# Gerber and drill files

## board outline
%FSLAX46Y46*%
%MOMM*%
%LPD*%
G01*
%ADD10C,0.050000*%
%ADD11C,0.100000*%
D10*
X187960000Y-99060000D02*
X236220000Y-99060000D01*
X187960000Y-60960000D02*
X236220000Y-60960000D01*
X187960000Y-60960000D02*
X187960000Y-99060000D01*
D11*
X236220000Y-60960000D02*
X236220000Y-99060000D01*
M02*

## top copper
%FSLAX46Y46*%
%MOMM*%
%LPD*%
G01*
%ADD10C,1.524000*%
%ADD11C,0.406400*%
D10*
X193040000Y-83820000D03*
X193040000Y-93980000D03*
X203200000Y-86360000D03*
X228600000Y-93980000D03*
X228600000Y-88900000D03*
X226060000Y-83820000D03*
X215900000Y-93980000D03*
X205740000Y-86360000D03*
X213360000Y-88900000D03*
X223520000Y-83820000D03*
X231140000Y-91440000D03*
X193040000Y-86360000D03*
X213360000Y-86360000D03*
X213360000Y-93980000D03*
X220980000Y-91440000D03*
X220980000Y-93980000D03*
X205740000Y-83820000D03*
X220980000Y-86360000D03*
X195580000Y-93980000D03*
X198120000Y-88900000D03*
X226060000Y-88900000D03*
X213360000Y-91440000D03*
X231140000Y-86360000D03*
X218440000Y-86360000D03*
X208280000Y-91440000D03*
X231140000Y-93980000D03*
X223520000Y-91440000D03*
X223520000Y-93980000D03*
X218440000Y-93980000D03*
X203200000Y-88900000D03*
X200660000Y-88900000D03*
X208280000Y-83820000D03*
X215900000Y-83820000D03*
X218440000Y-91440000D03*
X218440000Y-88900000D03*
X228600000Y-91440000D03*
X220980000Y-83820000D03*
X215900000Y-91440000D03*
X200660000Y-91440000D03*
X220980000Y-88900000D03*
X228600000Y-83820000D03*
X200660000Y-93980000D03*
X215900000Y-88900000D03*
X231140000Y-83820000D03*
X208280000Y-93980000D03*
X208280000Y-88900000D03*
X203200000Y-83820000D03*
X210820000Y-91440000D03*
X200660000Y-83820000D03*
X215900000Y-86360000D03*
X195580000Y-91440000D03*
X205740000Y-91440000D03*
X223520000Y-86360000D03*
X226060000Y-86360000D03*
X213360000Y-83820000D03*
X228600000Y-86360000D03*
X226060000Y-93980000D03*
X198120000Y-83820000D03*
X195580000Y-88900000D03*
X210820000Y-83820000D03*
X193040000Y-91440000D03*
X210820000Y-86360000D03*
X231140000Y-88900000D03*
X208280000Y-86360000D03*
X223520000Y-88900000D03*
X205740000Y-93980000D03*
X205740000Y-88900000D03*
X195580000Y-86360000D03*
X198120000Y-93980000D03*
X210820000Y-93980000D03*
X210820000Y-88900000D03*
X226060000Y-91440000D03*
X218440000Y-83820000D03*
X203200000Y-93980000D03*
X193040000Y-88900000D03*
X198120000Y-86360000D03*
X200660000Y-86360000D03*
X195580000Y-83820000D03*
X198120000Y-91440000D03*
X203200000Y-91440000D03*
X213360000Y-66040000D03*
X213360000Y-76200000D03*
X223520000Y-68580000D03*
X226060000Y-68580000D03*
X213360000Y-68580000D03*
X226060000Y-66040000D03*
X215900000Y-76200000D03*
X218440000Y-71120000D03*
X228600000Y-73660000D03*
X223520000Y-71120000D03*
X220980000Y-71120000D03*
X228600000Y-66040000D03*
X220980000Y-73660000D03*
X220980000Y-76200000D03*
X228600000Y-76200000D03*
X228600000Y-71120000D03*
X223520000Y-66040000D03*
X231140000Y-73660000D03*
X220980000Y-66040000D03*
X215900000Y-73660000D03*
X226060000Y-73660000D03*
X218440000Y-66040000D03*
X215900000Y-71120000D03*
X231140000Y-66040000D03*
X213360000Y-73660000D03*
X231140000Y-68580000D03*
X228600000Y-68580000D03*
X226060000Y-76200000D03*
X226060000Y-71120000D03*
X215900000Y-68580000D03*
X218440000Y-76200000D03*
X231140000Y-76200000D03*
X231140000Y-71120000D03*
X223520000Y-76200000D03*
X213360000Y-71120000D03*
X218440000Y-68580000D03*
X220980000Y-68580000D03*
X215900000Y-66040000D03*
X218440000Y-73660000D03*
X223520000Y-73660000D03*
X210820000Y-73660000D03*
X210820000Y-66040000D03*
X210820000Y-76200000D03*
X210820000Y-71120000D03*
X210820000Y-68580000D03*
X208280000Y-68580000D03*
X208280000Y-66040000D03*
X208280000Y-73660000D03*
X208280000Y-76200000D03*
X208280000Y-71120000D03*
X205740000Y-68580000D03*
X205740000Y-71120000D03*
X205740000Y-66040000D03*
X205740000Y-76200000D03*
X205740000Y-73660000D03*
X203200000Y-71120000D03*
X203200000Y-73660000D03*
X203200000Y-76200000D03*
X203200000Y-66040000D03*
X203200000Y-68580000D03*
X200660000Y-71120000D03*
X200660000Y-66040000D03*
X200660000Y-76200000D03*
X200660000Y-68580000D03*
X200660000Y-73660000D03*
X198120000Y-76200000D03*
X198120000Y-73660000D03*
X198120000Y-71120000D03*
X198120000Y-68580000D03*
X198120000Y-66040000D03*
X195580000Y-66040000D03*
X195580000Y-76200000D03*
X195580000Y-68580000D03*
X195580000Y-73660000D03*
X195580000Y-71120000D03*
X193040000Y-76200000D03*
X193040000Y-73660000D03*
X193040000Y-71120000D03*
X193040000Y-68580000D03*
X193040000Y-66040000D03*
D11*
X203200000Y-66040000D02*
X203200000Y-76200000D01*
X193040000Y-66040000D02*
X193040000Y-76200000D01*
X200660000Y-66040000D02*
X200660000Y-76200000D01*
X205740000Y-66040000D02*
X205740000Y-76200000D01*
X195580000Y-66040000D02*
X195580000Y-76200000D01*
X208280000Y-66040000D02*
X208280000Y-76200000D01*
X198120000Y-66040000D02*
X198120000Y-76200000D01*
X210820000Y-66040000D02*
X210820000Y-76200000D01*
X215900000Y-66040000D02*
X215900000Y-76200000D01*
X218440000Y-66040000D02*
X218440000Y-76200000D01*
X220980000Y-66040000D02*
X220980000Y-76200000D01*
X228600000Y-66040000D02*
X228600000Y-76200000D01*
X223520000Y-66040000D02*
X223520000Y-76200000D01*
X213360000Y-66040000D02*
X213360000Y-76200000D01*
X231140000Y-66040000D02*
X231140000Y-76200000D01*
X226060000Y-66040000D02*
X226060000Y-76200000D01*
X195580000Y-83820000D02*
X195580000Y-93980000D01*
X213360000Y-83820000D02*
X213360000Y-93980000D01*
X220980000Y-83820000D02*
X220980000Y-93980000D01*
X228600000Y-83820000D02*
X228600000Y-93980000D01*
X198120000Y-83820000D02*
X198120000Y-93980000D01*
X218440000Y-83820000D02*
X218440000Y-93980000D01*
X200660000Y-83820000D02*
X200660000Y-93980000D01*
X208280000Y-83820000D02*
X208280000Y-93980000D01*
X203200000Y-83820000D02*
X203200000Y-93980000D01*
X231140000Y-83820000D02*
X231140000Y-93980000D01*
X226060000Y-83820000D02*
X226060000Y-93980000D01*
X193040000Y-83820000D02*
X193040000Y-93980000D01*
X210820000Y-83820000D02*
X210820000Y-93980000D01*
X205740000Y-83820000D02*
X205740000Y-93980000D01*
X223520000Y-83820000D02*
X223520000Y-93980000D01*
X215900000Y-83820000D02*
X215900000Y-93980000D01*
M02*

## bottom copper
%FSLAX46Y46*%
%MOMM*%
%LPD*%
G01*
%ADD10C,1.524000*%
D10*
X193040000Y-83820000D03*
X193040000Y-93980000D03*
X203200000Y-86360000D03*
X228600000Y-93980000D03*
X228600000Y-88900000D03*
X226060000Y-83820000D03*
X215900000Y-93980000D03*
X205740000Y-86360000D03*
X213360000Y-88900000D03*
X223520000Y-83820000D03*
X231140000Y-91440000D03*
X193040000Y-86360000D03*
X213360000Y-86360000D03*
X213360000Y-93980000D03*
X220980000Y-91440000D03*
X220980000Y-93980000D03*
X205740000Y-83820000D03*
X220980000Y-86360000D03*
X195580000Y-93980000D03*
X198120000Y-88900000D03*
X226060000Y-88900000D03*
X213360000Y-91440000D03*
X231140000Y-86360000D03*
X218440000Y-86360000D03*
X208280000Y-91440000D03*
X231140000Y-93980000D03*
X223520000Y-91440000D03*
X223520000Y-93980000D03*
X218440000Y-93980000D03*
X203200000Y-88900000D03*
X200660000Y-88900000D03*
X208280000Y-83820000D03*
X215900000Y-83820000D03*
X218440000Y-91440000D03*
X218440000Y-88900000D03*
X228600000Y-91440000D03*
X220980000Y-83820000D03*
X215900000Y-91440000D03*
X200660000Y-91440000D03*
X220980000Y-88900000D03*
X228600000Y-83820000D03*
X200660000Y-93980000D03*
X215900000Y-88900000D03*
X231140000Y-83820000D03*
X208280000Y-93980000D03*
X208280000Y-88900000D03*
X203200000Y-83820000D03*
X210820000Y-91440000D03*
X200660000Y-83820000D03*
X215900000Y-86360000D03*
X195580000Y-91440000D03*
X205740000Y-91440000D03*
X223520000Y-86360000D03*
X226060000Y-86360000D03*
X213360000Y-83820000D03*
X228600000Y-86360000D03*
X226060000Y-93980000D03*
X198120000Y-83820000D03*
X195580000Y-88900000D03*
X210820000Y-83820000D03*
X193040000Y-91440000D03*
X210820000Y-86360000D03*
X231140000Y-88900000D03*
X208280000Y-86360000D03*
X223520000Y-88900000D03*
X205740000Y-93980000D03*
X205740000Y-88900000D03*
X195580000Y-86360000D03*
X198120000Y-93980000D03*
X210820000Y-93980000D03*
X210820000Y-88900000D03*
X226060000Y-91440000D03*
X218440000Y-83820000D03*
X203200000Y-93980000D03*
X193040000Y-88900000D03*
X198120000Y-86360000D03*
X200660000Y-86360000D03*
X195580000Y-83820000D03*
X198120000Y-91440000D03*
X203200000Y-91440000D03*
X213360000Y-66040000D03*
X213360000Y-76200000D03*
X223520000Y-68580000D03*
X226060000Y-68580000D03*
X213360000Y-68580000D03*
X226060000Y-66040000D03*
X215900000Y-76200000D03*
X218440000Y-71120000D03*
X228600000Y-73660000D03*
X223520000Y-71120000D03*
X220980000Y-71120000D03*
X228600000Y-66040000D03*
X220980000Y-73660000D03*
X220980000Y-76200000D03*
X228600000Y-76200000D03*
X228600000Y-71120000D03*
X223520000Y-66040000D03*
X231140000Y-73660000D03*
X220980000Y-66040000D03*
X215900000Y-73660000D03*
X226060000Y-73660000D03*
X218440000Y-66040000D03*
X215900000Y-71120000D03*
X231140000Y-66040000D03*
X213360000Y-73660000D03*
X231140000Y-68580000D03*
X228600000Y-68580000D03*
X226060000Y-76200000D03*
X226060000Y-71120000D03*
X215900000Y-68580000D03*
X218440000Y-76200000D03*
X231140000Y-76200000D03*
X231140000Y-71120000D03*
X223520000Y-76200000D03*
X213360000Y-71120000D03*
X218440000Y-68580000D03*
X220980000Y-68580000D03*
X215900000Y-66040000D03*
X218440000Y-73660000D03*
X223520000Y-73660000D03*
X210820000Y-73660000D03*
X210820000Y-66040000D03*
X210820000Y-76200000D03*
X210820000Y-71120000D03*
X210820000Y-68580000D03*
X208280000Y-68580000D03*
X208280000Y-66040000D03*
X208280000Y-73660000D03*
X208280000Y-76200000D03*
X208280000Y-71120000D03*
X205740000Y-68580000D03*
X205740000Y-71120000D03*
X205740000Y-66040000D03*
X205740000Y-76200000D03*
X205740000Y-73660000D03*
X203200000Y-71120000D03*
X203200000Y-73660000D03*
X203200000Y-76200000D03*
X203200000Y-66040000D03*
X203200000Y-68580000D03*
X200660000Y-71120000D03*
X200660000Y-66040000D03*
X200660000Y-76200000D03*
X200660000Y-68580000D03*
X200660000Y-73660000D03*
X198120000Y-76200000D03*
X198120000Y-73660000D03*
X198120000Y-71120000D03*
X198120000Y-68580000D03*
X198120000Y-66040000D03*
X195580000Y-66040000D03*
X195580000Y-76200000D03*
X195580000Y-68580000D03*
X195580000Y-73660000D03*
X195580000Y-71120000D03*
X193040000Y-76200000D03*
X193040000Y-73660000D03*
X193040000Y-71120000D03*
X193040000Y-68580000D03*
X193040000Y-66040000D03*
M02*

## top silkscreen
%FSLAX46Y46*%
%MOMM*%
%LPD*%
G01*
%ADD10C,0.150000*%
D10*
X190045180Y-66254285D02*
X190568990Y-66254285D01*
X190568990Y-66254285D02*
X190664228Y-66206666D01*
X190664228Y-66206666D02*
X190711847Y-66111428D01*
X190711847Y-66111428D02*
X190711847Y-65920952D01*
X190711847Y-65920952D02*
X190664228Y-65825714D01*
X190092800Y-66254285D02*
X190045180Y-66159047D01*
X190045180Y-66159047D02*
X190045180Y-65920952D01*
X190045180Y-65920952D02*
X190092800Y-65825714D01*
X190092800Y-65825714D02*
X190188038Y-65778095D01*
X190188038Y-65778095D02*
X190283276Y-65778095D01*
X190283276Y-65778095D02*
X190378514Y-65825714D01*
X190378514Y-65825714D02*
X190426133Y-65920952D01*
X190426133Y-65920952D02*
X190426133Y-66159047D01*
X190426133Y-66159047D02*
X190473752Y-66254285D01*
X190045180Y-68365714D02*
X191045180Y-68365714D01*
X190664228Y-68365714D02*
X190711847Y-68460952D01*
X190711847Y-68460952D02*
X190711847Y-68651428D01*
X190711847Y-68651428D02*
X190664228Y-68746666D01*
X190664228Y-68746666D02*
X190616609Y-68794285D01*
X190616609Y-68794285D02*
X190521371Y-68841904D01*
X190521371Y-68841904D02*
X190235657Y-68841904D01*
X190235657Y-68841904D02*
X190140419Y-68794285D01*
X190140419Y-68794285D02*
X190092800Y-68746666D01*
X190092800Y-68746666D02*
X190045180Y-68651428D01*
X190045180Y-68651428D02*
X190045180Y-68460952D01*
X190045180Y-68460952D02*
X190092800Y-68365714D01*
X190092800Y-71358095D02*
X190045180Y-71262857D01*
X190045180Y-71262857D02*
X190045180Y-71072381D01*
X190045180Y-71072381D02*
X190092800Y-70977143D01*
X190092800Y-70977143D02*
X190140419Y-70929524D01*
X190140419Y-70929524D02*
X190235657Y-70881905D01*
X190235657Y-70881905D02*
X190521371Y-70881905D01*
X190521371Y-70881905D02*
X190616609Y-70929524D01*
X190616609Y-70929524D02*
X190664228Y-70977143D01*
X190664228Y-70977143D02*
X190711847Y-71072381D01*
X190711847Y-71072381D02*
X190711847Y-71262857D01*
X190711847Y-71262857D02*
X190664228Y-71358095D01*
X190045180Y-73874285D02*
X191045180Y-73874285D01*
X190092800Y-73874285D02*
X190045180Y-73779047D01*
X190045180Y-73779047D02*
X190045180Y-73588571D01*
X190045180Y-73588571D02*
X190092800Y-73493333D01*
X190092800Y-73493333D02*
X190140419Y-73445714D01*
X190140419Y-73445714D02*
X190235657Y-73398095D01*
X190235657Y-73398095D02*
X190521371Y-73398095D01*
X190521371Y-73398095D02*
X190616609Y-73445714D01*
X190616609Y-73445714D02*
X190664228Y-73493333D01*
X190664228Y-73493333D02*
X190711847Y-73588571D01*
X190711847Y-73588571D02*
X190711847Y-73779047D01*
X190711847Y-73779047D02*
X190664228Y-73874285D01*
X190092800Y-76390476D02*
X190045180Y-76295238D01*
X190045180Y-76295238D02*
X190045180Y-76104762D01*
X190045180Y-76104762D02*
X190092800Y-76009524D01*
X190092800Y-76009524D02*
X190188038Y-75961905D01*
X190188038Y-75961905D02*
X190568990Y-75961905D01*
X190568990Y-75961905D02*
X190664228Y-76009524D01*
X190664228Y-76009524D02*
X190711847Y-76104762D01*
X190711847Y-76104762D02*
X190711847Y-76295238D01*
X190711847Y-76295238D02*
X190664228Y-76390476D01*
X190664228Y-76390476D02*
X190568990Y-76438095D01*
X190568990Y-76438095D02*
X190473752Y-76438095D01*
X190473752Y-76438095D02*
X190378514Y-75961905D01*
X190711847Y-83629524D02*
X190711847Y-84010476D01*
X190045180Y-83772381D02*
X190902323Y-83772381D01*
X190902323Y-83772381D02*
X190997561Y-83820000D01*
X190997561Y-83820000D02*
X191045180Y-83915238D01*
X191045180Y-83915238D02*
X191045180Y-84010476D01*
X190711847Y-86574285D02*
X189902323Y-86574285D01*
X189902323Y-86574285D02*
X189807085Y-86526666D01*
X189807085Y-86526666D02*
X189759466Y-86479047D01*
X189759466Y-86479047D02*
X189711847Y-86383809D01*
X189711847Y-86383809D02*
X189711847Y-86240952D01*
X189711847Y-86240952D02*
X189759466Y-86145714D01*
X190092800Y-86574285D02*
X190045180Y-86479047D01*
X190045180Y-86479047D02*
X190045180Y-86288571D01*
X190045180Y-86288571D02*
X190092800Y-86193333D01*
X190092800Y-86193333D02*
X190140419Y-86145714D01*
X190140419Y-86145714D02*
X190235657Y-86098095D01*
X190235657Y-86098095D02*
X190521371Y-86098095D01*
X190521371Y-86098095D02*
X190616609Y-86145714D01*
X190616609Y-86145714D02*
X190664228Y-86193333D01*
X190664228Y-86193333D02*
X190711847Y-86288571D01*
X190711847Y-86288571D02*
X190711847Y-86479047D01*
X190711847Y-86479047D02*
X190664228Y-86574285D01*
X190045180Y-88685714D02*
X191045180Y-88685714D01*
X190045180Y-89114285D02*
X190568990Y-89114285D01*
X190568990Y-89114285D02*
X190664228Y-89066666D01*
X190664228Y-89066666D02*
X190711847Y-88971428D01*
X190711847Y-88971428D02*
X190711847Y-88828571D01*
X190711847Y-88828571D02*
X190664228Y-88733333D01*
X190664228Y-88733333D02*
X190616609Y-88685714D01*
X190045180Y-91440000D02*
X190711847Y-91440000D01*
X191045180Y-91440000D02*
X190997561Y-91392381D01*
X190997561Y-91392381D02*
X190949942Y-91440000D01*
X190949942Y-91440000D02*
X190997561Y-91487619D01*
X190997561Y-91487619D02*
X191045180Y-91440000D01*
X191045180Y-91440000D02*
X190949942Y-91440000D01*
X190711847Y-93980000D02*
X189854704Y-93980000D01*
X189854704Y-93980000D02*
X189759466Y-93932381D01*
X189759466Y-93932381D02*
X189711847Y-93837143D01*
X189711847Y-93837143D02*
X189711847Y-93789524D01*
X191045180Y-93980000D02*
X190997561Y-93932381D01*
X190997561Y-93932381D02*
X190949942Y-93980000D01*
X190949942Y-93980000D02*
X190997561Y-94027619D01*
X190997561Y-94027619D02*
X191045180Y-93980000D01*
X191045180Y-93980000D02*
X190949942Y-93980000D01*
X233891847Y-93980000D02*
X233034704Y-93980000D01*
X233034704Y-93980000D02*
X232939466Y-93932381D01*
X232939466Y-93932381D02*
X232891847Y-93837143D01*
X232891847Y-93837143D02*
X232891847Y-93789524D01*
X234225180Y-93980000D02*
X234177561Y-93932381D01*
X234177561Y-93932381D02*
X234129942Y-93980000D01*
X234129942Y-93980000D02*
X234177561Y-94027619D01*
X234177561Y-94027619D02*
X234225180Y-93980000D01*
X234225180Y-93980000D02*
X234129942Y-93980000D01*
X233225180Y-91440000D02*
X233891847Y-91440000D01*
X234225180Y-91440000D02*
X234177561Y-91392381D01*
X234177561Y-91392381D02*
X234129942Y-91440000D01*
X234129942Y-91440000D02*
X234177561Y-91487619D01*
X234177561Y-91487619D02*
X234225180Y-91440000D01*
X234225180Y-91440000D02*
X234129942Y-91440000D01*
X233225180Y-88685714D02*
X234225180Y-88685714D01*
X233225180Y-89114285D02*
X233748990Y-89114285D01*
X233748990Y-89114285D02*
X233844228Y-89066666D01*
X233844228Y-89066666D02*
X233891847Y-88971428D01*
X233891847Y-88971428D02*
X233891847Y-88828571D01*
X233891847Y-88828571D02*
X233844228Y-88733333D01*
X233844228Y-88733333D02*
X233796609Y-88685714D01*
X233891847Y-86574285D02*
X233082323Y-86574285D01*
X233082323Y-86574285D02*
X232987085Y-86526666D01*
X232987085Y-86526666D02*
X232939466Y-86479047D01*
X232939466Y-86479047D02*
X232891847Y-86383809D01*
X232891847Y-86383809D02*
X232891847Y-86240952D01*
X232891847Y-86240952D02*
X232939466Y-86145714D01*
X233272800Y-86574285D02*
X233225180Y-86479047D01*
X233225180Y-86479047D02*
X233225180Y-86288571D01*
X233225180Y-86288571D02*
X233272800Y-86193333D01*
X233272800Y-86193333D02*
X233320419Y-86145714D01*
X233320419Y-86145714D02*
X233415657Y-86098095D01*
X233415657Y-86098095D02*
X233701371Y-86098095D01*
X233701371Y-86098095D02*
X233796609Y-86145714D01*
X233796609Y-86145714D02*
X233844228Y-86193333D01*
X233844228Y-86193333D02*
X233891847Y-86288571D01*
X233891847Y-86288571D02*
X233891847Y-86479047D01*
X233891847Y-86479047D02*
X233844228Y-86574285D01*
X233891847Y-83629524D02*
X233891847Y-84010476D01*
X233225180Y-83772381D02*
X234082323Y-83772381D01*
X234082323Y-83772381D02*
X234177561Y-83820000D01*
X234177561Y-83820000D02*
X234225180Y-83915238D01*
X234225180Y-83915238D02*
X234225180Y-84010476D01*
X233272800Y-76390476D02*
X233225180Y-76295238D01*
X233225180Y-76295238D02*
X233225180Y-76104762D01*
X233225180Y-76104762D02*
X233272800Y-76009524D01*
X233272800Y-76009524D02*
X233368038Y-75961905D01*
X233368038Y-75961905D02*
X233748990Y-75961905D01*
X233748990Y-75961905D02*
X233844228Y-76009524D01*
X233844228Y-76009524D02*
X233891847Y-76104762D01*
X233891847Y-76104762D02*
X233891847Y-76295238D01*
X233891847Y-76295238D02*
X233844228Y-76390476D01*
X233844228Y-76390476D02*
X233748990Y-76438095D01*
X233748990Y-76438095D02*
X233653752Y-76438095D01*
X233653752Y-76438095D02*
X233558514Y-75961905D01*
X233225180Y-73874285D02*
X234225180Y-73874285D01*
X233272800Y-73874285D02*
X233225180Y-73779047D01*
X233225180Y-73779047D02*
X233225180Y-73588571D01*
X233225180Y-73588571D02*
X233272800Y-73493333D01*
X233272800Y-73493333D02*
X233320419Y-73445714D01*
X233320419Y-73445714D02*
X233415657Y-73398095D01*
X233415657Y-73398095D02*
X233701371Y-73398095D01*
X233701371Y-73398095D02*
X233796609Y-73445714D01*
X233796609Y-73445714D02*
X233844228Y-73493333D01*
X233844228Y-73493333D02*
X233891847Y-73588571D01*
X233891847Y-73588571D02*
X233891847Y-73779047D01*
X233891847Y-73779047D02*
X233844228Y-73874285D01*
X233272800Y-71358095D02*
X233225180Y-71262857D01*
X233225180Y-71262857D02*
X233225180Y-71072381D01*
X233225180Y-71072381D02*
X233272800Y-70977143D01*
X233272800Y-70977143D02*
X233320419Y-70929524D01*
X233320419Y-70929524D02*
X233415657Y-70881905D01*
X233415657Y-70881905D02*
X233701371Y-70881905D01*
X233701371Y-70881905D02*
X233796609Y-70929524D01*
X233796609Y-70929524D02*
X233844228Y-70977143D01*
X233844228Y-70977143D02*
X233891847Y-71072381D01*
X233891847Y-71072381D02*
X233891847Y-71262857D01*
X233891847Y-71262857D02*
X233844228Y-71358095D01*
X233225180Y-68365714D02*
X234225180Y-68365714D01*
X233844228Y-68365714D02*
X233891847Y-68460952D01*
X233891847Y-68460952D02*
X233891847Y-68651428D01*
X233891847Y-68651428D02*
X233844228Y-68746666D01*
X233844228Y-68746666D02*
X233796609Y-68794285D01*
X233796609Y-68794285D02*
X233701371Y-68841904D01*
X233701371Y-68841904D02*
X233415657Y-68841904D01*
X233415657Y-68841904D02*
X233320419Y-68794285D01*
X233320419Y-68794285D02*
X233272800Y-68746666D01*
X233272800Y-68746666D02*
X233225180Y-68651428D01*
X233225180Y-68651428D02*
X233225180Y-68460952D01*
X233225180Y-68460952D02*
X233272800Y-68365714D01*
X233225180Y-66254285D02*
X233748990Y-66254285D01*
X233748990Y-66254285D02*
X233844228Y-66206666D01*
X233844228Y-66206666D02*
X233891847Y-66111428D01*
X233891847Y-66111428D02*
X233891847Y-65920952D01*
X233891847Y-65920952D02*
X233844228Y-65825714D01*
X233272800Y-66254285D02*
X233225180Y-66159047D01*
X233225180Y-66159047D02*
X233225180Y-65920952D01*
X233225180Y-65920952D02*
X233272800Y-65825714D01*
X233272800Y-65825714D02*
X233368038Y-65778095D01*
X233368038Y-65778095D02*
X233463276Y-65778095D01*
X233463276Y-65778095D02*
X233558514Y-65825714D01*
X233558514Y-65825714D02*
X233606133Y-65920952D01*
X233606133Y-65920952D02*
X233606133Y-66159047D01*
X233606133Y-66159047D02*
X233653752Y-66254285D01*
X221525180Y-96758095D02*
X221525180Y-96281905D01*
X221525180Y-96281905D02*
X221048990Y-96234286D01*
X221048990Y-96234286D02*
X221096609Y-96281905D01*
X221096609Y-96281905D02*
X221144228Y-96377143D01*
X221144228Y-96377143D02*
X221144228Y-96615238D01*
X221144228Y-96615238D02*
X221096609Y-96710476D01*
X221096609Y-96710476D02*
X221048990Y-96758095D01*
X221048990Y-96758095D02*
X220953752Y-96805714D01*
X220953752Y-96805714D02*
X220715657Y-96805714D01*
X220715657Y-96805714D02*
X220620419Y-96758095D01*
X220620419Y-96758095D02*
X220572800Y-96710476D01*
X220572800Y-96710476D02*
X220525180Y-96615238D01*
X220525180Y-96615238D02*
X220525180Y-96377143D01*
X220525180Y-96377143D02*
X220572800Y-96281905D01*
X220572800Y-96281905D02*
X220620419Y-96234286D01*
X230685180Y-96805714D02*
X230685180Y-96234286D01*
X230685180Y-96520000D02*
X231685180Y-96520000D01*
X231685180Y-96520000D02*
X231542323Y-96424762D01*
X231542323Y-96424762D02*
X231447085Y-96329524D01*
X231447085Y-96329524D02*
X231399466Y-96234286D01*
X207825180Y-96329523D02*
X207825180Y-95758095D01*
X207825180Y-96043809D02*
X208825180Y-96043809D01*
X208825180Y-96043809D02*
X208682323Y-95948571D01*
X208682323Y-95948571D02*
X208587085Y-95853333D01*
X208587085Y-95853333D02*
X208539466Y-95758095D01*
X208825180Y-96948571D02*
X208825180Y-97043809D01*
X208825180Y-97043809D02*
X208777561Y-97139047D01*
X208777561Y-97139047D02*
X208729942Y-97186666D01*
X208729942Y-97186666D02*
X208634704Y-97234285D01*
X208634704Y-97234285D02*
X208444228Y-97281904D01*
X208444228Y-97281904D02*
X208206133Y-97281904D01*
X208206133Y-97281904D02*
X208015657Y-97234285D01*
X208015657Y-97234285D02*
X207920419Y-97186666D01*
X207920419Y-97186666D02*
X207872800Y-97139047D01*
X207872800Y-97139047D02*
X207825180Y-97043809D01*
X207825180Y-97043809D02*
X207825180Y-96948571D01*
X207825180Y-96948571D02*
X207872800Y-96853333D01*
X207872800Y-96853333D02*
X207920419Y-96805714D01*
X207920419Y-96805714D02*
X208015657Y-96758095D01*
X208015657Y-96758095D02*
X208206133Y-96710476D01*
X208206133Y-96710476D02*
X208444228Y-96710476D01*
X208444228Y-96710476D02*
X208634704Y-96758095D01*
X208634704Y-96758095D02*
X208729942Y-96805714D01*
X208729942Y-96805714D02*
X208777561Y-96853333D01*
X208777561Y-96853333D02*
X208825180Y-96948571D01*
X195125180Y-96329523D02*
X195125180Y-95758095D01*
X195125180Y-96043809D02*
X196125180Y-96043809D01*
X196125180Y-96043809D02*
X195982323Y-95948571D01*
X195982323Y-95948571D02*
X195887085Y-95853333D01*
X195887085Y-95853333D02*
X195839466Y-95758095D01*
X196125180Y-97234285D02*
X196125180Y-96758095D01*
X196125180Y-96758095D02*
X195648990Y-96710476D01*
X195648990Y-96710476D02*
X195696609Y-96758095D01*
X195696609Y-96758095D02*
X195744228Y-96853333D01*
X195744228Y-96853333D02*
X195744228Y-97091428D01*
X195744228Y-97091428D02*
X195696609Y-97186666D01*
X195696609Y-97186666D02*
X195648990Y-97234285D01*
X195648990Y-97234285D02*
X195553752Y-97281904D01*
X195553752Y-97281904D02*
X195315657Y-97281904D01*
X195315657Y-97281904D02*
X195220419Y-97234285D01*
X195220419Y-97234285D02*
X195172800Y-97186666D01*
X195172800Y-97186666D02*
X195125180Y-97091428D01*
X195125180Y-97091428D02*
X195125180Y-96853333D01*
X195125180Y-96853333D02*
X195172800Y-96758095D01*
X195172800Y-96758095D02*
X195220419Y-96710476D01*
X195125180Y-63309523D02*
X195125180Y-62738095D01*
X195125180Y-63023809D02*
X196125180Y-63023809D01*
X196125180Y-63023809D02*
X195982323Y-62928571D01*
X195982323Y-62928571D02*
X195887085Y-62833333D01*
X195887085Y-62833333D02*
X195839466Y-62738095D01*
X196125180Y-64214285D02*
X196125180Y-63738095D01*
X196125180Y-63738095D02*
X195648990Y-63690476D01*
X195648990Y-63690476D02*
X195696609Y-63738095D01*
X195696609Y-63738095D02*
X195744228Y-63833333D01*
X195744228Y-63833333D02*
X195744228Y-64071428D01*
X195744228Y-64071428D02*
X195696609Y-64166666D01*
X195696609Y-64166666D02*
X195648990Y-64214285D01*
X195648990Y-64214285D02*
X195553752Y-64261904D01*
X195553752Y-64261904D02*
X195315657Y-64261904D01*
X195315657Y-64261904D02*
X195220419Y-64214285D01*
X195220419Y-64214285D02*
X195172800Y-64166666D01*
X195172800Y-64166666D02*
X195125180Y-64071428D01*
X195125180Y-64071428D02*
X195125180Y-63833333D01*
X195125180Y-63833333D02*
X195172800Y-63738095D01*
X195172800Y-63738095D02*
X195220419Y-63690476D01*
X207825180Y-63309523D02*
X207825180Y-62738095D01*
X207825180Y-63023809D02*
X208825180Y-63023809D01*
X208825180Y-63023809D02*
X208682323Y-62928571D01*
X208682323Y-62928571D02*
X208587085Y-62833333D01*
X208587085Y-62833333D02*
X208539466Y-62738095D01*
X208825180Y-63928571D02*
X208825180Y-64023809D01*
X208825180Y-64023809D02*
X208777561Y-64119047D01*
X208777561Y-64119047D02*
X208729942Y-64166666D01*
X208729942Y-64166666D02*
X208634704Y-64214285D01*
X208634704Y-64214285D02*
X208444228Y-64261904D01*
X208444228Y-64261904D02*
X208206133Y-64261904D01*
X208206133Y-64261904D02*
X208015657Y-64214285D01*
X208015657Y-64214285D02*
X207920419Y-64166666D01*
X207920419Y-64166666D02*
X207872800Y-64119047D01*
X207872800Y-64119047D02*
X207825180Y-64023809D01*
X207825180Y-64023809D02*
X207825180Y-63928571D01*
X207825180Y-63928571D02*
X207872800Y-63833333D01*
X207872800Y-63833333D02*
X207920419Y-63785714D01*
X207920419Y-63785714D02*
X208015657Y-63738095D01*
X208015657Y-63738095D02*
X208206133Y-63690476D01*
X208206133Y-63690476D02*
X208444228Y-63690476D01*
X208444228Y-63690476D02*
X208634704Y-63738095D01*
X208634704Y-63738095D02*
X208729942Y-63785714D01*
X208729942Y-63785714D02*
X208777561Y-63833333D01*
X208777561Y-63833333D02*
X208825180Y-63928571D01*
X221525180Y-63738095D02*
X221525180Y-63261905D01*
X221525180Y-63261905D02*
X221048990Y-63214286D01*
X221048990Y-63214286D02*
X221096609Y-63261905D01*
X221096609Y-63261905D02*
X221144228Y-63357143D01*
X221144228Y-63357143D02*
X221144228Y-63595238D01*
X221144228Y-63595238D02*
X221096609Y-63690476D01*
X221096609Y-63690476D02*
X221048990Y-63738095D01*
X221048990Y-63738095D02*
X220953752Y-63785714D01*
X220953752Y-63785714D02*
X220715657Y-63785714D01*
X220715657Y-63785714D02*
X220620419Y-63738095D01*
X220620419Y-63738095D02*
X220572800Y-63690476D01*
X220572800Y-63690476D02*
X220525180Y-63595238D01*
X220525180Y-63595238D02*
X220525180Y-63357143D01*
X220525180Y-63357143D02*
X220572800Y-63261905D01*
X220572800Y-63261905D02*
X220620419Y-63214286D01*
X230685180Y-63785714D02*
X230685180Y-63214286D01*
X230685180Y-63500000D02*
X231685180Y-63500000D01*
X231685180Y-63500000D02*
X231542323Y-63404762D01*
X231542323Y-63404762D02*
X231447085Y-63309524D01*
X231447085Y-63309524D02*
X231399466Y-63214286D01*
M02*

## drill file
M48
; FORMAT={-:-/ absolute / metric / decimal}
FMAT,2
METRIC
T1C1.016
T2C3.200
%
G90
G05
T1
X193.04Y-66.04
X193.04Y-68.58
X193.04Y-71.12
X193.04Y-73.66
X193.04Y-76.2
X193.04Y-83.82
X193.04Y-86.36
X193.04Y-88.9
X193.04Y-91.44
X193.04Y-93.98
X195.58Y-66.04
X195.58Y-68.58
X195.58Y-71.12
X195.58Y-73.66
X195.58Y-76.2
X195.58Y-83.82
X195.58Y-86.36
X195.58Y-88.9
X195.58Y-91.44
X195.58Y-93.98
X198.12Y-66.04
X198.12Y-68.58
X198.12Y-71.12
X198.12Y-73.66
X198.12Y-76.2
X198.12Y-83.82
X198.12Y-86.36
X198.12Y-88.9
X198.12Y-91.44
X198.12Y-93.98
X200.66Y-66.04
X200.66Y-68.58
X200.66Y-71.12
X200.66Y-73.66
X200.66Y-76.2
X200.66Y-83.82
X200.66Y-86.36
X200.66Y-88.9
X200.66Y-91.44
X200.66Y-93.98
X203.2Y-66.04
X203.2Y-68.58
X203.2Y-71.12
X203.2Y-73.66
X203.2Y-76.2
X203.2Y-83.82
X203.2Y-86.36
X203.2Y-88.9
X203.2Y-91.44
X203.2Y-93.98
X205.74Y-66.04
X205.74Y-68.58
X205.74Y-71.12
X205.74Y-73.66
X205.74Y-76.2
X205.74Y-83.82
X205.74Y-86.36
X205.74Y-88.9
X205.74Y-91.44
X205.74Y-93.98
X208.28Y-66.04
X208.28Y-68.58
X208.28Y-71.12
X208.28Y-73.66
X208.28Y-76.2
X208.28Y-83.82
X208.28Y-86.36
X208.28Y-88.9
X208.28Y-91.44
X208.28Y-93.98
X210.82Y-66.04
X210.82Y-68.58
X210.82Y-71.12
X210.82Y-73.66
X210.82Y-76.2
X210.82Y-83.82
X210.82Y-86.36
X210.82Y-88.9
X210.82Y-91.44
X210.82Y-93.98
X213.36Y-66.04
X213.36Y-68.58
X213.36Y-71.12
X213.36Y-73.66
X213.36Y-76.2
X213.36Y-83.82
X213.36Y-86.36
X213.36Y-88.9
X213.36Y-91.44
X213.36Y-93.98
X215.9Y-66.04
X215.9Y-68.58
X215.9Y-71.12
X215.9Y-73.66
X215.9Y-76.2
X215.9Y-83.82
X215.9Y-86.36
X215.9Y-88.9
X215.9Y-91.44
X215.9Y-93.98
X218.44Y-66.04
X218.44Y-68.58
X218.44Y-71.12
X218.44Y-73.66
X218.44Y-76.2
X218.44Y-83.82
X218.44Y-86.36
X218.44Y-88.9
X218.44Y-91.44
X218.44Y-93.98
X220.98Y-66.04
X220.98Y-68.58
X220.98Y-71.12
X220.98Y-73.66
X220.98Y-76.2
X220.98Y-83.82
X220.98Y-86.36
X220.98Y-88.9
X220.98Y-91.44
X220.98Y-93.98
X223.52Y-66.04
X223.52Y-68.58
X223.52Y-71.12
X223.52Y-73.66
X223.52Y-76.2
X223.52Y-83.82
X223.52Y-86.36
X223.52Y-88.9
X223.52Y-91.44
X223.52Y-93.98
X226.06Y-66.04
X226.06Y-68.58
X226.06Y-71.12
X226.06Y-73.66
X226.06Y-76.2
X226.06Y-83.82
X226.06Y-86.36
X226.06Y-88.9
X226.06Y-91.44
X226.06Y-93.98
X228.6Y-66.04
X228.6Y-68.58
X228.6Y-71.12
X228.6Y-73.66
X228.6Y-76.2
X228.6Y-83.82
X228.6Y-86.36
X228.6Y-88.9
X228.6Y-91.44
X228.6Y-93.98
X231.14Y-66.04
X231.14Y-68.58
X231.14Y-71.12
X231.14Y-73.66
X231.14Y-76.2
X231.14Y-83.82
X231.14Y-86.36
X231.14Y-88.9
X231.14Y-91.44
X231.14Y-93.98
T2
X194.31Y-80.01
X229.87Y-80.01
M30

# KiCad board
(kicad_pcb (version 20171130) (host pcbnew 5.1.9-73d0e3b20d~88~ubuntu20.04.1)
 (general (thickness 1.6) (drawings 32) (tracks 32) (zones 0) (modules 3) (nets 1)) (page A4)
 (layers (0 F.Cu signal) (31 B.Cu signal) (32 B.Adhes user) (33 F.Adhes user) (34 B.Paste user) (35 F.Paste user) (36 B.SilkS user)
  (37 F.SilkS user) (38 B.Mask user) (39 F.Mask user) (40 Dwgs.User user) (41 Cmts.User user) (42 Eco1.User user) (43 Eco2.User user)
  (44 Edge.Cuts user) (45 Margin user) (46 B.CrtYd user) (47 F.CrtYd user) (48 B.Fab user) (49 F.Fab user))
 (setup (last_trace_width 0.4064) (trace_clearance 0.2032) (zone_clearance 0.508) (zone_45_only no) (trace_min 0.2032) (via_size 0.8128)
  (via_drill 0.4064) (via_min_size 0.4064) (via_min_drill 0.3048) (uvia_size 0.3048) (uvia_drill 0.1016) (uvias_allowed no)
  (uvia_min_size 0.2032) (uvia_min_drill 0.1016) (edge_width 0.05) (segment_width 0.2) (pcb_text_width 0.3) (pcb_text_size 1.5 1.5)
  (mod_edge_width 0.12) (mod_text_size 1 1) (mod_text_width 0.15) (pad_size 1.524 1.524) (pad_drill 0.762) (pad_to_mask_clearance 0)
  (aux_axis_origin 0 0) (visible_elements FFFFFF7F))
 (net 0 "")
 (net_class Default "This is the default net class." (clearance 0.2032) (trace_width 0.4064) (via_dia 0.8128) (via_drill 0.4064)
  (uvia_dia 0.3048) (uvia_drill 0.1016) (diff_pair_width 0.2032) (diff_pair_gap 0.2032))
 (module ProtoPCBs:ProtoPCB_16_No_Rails (layer F.Cu) (at 193.04 66.04)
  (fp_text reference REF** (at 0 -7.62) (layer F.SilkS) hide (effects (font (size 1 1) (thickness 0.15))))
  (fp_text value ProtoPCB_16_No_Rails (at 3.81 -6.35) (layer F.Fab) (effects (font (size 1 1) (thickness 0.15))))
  (pad 1 thru_hole circle (at 0 17.78) (size 1.524 1.524) (drill 1.016) (layers *.Cu *.Mask))
  (pad 1 thru_hole circle (at 0 27.94) (size 1.524 1.524) (drill 1.016) (layers *.Cu *.Mask))
  (pad 1 thru_hole circle (at 10.16 20.32) (size 1.524 1.524) (drill 1.016) (layers *.Cu *.Mask))
  (pad 1 thru_hole circle (at 35.56 27.94) (size 1.524 1.524) (drill 1.016) (layers *.Cu *.Mask))
  (pad 1 thru_hole circle (at 35.56 22.86) (size 1.524 1.524) (drill 1.016) (layers *.Cu *.Mask))
  (pad 1 thru_hole circle (at 33.02 17.78) (size 1.524 1.524) (drill 1.016) (layers *.Cu *.Mask))
  (pad 1 thru_hole circle (at 22.86 27.94) (size 1.524 1.524) (drill 1.016) (layers *.Cu *.Mask))
  (pad 1 thru_hole circle (at 12.7 20.32) (size 1.524 1.524) (drill 1.016) (layers *.Cu *.Mask))
  (pad 1 thru_hole circle (at 20.32 22.86) (size 1.524 1.524) (drill 1.016) (layers *.Cu *.Mask))
  (pad 1 thru_hole circle (at 30.48 17.78) (size 1.524 1.524) (drill 1.016) (layers *.Cu *.Mask))
  (pad 1 thru_hole circle (at 38.1 25.4) (size 1.524 1.524) (drill 1.016) (layers *.Cu *.Mask))
  (pad 1 thru_hole circle (at 0 20.32) (size 1.524 1.524) (drill 1.016) (layers *.Cu *.Mask))
  (pad 1 thru_hole circle (at 20.32 20.32) (size 1.524 1.524) (drill 1.016) (layers *.Cu *.Mask))
  (pad 1 thru_hole circle (at 20.32 27.94) (size 1.524 1.524) (drill 1.016) (layers *.Cu *.Mask))
  (pad 1 thru_hole circle (at 27.94 25.4) (size 1.524 1.524) (drill 1.016) (layers *.Cu *.Mask))
  (pad 1 thru_hole circle (at 27.94 27.94) (size 1.524 1.524) (drill 1.016) (layers *.Cu *.Mask))
  (pad 1 thru_hole circle (at 12.7 17.78) (size 1.524 1.524) (drill 1.016) (layers *.Cu *.Mask))
  (pad 1 thru_hole circle (at 27.94 20.32) (size 1.524 1.524) (drill 1.016) (layers *.Cu *.Mask))
  (pad 1 thru_hole circle (at 2.54 27.94) (size 1.524 1.524) (drill 1.016) (layers *.Cu *.Mask))
  (pad 1 thru_hole circle (at 5.08 22.86) (size 1.524 1.524) (drill 1.016) (layers *.Cu *.Mask))
  (pad 1 thru_hole circle (at 33.02 22.86) (size 1.524 1.524) (drill 1.016) (layers *.Cu *.Mask))
  (pad 1 thru_hole circle (at 20.32 25.4) (size 1.524 1.524) (drill 1.016) (layers *.Cu *.Mask))
  (pad 1 thru_hole circle (at 38.1 20.32) (size 1.524 1.524) (drill 1.016) (layers *.Cu *.Mask))
  (pad 1 thru_hole circle (at 25.4 20.32) (size 1.524 1.524) (drill 1.016) (layers *.Cu *.Mask))
  (pad 1 thru_hole circle (at 15.24 25.4) (size 1.524 1.524) (drill 1.016) (layers *.Cu *.Mask))
  (pad 1 thru_hole circle (at 38.1 27.94) (size 1.524 1.524) (drill 1.016) (layers *.Cu *.Mask))
  (pad 1 thru_hole circle (at 30.48 25.4) (size 1.524 1.524) (drill 1.016) (layers *.Cu *.Mask))
  (pad 1 thru_hole circle (at 30.48 27.94) (size 1.524 1.524) (drill 1.016) (layers *.Cu *.Mask))
  (pad 1 thru_hole circle (at 25.4 27.94) (size 1.524 1.524) (drill 1.016) (layers *.Cu *.Mask))
  (pad 1 thru_hole circle (at 10.16 22.86) (size 1.524 1.524) (drill 1.016) (layers *.Cu *.Mask))
  (pad 1 thru_hole circle (at 7.62 22.86) (size 1.524 1.524) (drill 1.016) (layers *.Cu *.Mask))
  (pad 1 thru_hole circle (at 15.24 17.78) (size 1.524 1.524) (drill 1.016) (layers *.Cu *.Mask))
  (pad 1 thru_hole circle (at 22.86 17.78) (size 1.524 1.524) (drill 1.016) (layers *.Cu *.Mask))
  (pad 1 thru_hole circle (at 25.4 25.4) (size 1.524 1.524) (drill 1.016) (layers *.Cu *.Mask))
  (pad 1 thru_hole circle (at 25.4 22.86) (size 1.524 1.524) (drill 1.016) (layers *.Cu *.Mask))
  (pad 1 thru_hole circle (at 35.56 25.4) (size 1.524 1.524) (drill 1.016) (layers *.Cu *.Mask))
  (pad 1 thru_hole circle (at 27.94 17.78) (size 1.524 1.524) (drill 1.016) (layers *.Cu *.Mask))
  (pad 1 thru_hole circle (at 22.86 25.4) (size 1.524 1.524) (drill 1.016) (layers *.Cu *.Mask))
  (pad 1 thru_hole circle (at 7.62 25.4) (size 1.524 1.524) (drill 1.016) (layers *.Cu *.Mask))
  (pad 1 thru_hole circle (at 27.94 22.86) (size 1.524 1.524) (drill 1.016) (layers *.Cu *.Mask))
  (pad 1 thru_hole circle (at 35.56 17.78) (size 1.524 1.524) (drill 1.016) (layers *.Cu *.Mask))
  (pad 1 thru_hole circle (at 7.62 27.94) (size 1.524 1.524) (drill 1.016) (layers *.Cu *.Mask))
  (pad 1 thru_hole circle (at 22.86 22.86) (size 1.524 1.524) (drill 1.016) (layers *.Cu *.Mask))
  (pad 1 thru_hole circle (at 38.1 17.78) (size 1.524 1.524) (drill 1.016) (layers *.Cu *.Mask))
  (pad 1 thru_hole circle (at 15.24 27.94) (size 1.524 1.524) (drill 1.016) (layers *.Cu *.Mask))
  (pad 1 thru_hole circle (at 15.24 22.86) (size 1.524 1.524) (drill 1.016) (layers *.Cu *.Mask))
  (pad 1 thru_hole circle (at 10.16 17.78) (size 1.524 1.524) (drill 1.016) (layers *.Cu *.Mask))
  (pad 1 thru_hole circle (at 17.78 25.4) (size 1.524 1.524) (drill 1.016) (layers *.Cu *.Mask))
  (pad 1 thru_hole circle (at 7.62 17.78) (size 1.524 1.524) (drill 1.016) (layers *.Cu *.Mask))
  (pad 1 thru_hole circle (at 22.86 20.32) (size 1.524 1.524) (drill 1.016) (layers *.Cu *.Mask))
  (pad 1 thru_hole circle (at 2.54 25.4) (size 1.524 1.524) (drill 1.016) (layers *.Cu *.Mask))
  (pad 1 thru_hole circle (at 12.7 25.4) (size 1.524 1.524) (drill 1.016) (layers *.Cu *.Mask))
  (pad 1 thru_hole circle (at 30.48 20.32) (size 1.524 1.524) (drill 1.016) (layers *.Cu *.Mask))
  (pad 1 thru_hole circle (at 33.02 20.32) (size 1.524 1.524) (drill 1.016) (layers *.Cu *.Mask))
  (pad 1 thru_hole circle (at 20.32 17.78) (size 1.524 1.524) (drill 1.016) (layers *.Cu *.Mask))
  (pad 1 thru_hole circle (at 35.56 20.32) (size 1.524 1.524) (drill 1.016) (layers *.Cu *.Mask))
  (pad 1 thru_hole circle (at 33.02 27.94) (size 1.524 1.524) (drill 1.016) (layers *.Cu *.Mask))
  (pad 1 thru_hole circle (at 5.08 17.78) (size 1.524 1.524) (drill 1.016) (layers *.Cu *.Mask))
  (pad 1 thru_hole circle (at 2.54 22.86) (size 1.524 1.524) (drill 1.016) (layers *.Cu *.Mask))
  (pad 1 thru_hole circle (at 17.78 17.78) (size 1.524 1.524) (drill 1.016) (layers *.Cu *.Mask))
  (pad 1 thru_hole circle (at 0 25.4) (size 1.524 1.524) (drill 1.016) (layers *.Cu *.Mask))
  (pad 1 thru_hole circle (at 17.78 20.32) (size 1.524 1.524) (drill 1.016) (layers *.Cu *.Mask))
  (pad 1 thru_hole circle (at 38.1 22.86) (size 1.524 1.524) (drill 1.016) (layers *.Cu *.Mask))
  (pad 1 thru_hole circle (at 15.24 20.32) (size 1.524 1.524) (drill 1.016) (layers *.Cu *.Mask))
  (pad 1 thru_hole circle (at 30.48 22.86) (size 1.524 1.524) (drill 1.016) (layers *.Cu *.Mask))
  (pad 1 thru_hole circle (at 12.7 27.94) (size 1.524 1.524) (drill 1.016) (layers *.Cu *.Mask))
  (pad 1 thru_hole circle (at 12.7 22.86) (size 1.524 1.524) (drill 1.016) (layers *.Cu *.Mask))
  (pad 1 thru_hole circle (at 2.54 20.32) (size 1.524 1.524) (drill 1.016) (layers *.Cu *.Mask))
  (pad 1 thru_hole circle (at 5.08 27.94) (size 1.524 1.524) (drill 1.016) (layers *.Cu *.Mask))
  (pad 1 thru_hole circle (at 17.78 27.94) (size 1.524 1.524) (drill 1.016) (layers *.Cu *.Mask))
  (pad 1 thru_hole circle (at 17.78 22.86) (size 1.524 1.524) (drill 1.016) (layers *.Cu *.Mask))
  (pad 1 thru_hole circle (at 33.02 25.4) (size 1.524 1.524) (drill 1.016) (layers *.Cu *.Mask))
  (pad 1 thru_hole circle (at 25.4 17.78) (size 1.524 1.524) (drill 1.016) (layers *.Cu *.Mask))
  (pad 1 thru_hole circle (at 10.16 27.94) (size 1.524 1.524) (drill 1.016) (layers *.Cu *.Mask))
  (pad 1 thru_hole circle (at 0 22.86) (size 1.524 1.524) (drill 1.016) (layers *.Cu *.Mask))
  (pad 1 thru_hole circle (at 5.08 20.32) (size 1.524 1.524) (drill 1.016) (layers *.Cu *.Mask))
  (pad 1 thru_hole circle (at 7.62 20.32) (size 1.524 1.524) (drill 1.016) (layers *.Cu *.Mask))
  (pad 1 thru_hole circle (at 2.54 17.78) (size 1.524 1.524) (drill 1.016) (layers *.Cu *.Mask))
  (pad 1 thru_hole circle (at 5.08 25.4) (size 1.524 1.524) (drill 1.016) (layers *.Cu *.Mask))
  (pad 1 thru_hole circle (at 10.16 25.4) (size 1.524 1.524) (drill 1.016) (layers *.Cu *.Mask))
  (pad 1 thru_hole circle (at 20.32 0) (size 1.524 1.524) (drill 1.016) (layers *.Cu *.Mask))
  (pad 1 thru_hole circle (at 20.32 10.16) (size 1.524 1.524) (drill 1.016) (layers *.Cu *.Mask))
  (pad 1 thru_hole circle (at 30.48 2.54) (size 1.524 1.524) (drill 1.016) (layers *.Cu *.Mask))
  (pad 1 thru_hole circle (at 33.02 2.54) (size 1.524 1.524) (drill 1.016) (layers *.Cu *.Mask))
  (pad 1 thru_hole circle (at 20.32 2.54) (size 1.524 1.524) (drill 1.016) (layers *.Cu *.Mask))
  (pad 1 thru_hole circle (at 33.02 0) (size 1.524 1.524) (drill 1.016) (layers *.Cu *.Mask))
  (pad 1 thru_hole circle (at 22.86 10.16) (size 1.524 1.524) (drill 1.016) (layers *.Cu *.Mask))
  (pad 1 thru_hole circle (at 25.4 5.08) (size 1.524 1.524) (drill 1.016) (layers *.Cu *.Mask))
  (pad 1 thru_hole circle (at 35.56 7.62) (size 1.524 1.524) (drill 1.016) (layers *.Cu *.Mask))
  (pad 1 thru_hole circle (at 30.48 5.08) (size 1.524 1.524) (drill 1.016) (layers *.Cu *.Mask))
  (pad 1 thru_hole circle (at 27.94 5.08) (size 1.524 1.524) (drill 1.016) (layers *.Cu *.Mask))
  (pad 1 thru_hole circle (at 35.56 0) (size 1.524 1.524) (drill 1.016) (layers *.Cu *.Mask))
  (pad 1 thru_hole circle (at 27.94 7.62) (size 1.524 1.524) (drill 1.016) (layers *.Cu *.Mask))
  (pad 1 thru_hole circle (at 27.94 10.16) (size 1.524 1.524) (drill 1.016) (layers *.Cu *.Mask))
  (pad 1 thru_hole circle (at 35.56 10.16) (size 1.524 1.524) (drill 1.016) (layers *.Cu *.Mask))
  (pad 1 thru_hole circle (at 35.56 5.08) (size 1.524 1.524) (drill 1.016) (layers *.Cu *.Mask))
  (pad 1 thru_hole circle (at 30.48 0) (size 1.524 1.524) (drill 1.016) (layers *.Cu *.Mask))
  (pad 1 thru_hole circle (at 38.1 7.62) (size 1.524 1.524) (drill 1.016) (layers *.Cu *.Mask))
  (pad 1 thru_hole circle (at 27.94 0) (size 1.524 1.524) (drill 1.016) (layers *.Cu *.Mask))
  (pad 1 thru_hole circle (at 22.86 7.62) (size 1.524 1.524) (drill 1.016) (layers *.Cu *.Mask))
  (pad 1 thru_hole circle (at 33.02 7.62) (size 1.524 1.524) (drill 1.016) (layers *.Cu *.Mask))
  (pad 1 thru_hole circle (at 25.4 0) (size 1.524 1.524) (drill 1.016) (layers *.Cu *.Mask))
  (pad 1 thru_hole circle (at 22.86 5.08) (size 1.524 1.524) (drill 1.016) (layers *.Cu *.Mask))
  (pad 1 thru_hole circle (at 38.1 0) (size 1.524 1.524) (drill 1.016) (layers *.Cu *.Mask))
  (pad 1 thru_hole circle (at 20.32 7.62) (size 1.524 1.524) (drill 1.016) (layers *.Cu *.Mask))
  (pad 1 thru_hole circle (at 38.1 2.54) (size 1.524 1.524) (drill 1.016) (layers *.Cu *.Mask))
  (pad 1 thru_hole circle (at 35.56 2.54) (size 1.524 1.524) (drill 1.016) (layers *.Cu *.Mask))
  (pad 1 thru_hole circle (at 33.02 10.16) (size 1.524 1.524) (drill 1.016) (layers *.Cu *.Mask))
  (pad 1 thru_hole circle (at 33.02 5.08) (size 1.524 1.524) (drill 1.016) (layers *.Cu *.Mask))
  (pad 1 thru_hole circle (at 22.86 2.54) (size 1.524 1.524) (drill 1.016) (layers *.Cu *.Mask))
  (pad 1 thru_hole circle (at 25.4 10.16) (size 1.524 1.524) (drill 1.016) (layers *.Cu *.Mask))
  (pad 1 thru_hole circle (at 38.1 10.16) (size 1.524 1.524) (drill 1.016) (layers *.Cu *.Mask))
  (pad 1 thru_hole circle (at 38.1 5.08) (size 1.524 1.524) (drill 1.016) (layers *.Cu *.Mask))
  (pad 1 thru_hole circle (at 30.48 10.16) (size 1.524 1.524) (drill 1.016) (layers *.Cu *.Mask))
  (pad 1 thru_hole circle (at 20.32 5.08) (size 1.524 1.524) (drill 1.016) (layers *.Cu *.Mask))
  (pad 1 thru_hole circle (at 25.4 2.54) (size 1.524 1.524) (drill 1.016) (layers *.Cu *.Mask))
  (pad 1 thru_hole circle (at 27.94 2.54) (size 1.524 1.524) (drill 1.016) (layers *.Cu *.Mask))
  (pad 1 thru_hole circle (at 22.86 0) (size 1.524 1.524) (drill 1.016) (layers *.Cu *.Mask))
  (pad 1 thru_hole circle (at 25.4 7.62) (size 1.524 1.524) (drill 1.016) (layers *.Cu *.Mask))
  (pad 1 thru_hole circle (at 30.48 7.62) (size 1.524 1.524) (drill 1.016) (layers *.Cu *.Mask))
  (pad 1 thru_hole circle (at 17.78 7.62) (size 1.524 1.524) (drill 1.016) (layers *.Cu *.Mask))
  (pad 1 thru_hole circle (at 17.78 0) (size 1.524 1.524) (drill 1.016) (layers *.Cu *.Mask))
  (pad 1 thru_hole circle (at 17.78 10.16) (size 1.524 1.524) (drill 1.016) (layers *.Cu *.Mask))
  (pad 1 thru_hole circle (at 17.78 5.08) (size 1.524 1.524) (drill 1.016) (layers *.Cu *.Mask))
  (pad 1 thru_hole circle (at 17.78 2.54) (size 1.524 1.524) (drill 1.016) (layers *.Cu *.Mask))
  (pad 1 thru_hole circle (at 15.24 2.54) (size 1.524 1.524) (drill 1.016) (layers *.Cu *.Mask))
  (pad 1 thru_hole circle (at 15.24 0) (size 1.524 1.524) (drill 1.016) (layers *.Cu *.Mask))
  (pad 1 thru_hole circle (at 15.24 7.62) (size 1.524 1.524) (drill 1.016) (layers *.Cu *.Mask))
  (pad 1 thru_hole circle (at 15.24 10.16) (size 1.524 1.524) (drill 1.016) (layers *.Cu *.Mask))
  (pad 1 thru_hole circle (at 15.24 5.08) (size 1.524 1.524) (drill 1.016) (layers *.Cu *.Mask))
  (pad 1 thru_hole circle (at 12.7 2.54) (size 1.524 1.524) (drill 1.016) (layers *.Cu *.Mask))
  (pad 1 thru_hole circle (at 12.7 5.08) (size 1.524 1.524) (drill 1.016) (layers *.Cu *.Mask))
  (pad 1 thru_hole circle (at 12.7 0) (size 1.524 1.524) (drill 1.016) (layers *.Cu *.Mask))
  (pad 1 thru_hole circle (at 12.7 10.16) (size 1.524 1.524) (drill 1.016) (layers *.Cu *.Mask))
  (pad 1 thru_hole circle (at 12.7 7.62) (size 1.524 1.524) (drill 1.016) (layers *.Cu *.Mask))
  (pad 1 thru_hole circle (at 10.16 5.08) (size 1.524 1.524) (drill 1.016) (layers *.Cu *.Mask))
  (pad 1 thru_hole circle (at 10.16 7.62) (size 1.524 1.524) (drill 1.016) (layers *.Cu *.Mask))
  (pad 1 thru_hole circle (at 10.16 10.16) (size 1.524 1.524) (drill 1.016) (layers *.Cu *.Mask))
  (pad 1 thru_hole circle (at 10.16 0) (size 1.524 1.524) (drill 1.016) (layers *.Cu *.Mask))
  (pad 1 thru_hole circle (at 10.16 2.54) (size 1.524 1.524) (drill 1.016) (layers *.Cu *.Mask))
  (pad 1 thru_hole circle (at 7.62 5.08) (size 1.524 1.524) (drill 1.016) (layers *.Cu *.Mask))
  (pad 1 thru_hole circle (at 7.62 0) (size 1.524 1.524) (drill 1.016) (layers *.Cu *.Mask))
  (pad 1 thru_hole circle (at 7.62 10.16) (size 1.524 1.524) (drill 1.016) (layers *.Cu *.Mask))
  (pad 1 thru_hole circle (at 7.62 2.54) (size 1.524 1.524) (drill 1.016) (layers *.Cu *.Mask))
  (pad 1 thru_hole circle (at 7.62 7.62) (size 1.524 1.524) (drill 1.016) (layers *.Cu *.Mask))
  (pad 1 thru_hole circle (at 5.08 10.16) (size 1.524 1.524) (drill 1.016) (layers *.Cu *.Mask))
  (pad 1 thru_hole circle (at 5.08 7.62) (size 1.524 1.524) (drill 1.016) (layers *.Cu *.Mask))
  (pad 1 thru_hole circle (at 5.08 5.08) (size 1.524 1.524) (drill 1.016) (layers *.Cu *.Mask))
  (pad 1 thru_hole circle (at 5.08 2.54) (size 1.524 1.524) (drill 1.016) (layers *.Cu *.Mask))
  (pad 1 thru_hole circle (at 5.08 0) (size 1.524 1.524) (drill 1.016) (layers *.Cu *.Mask))
  (pad 1 thru_hole circle (at 2.54 0) (size 1.524 1.524) (drill 1.016) (layers *.Cu *.Mask))
  (pad 1 thru_hole circle (at 2.54 10.16) (size 1.524 1.524) (drill 1.016) (layers *.Cu *.Mask))
  (pad 1 thru_hole circle (at 2.54 2.54) (size 1.524 1.524) (drill 1.016) (layers *.Cu *.Mask))
  (pad 1 thru_hole circle (at 2.54 7.62) (size 1.524 1.524) (drill 1.016) (layers *.Cu *.Mask))
  (pad 1 thru_hole circle (at 2.54 5.08) (size 1.524 1.524) (drill 1.016) (layers *.Cu *.Mask))
  (pad 1 thru_hole circle (at 0 10.16) (size 1.524 1.524) (drill 1.016) (layers *.Cu *.Mask))
  (pad 1 thru_hole circle (at 0 7.62) (size 1.524 1.524) (drill 1.016) (layers *.Cu *.Mask))
  (pad 1 thru_hole circle (at 0 5.08) (size 1.524 1.524) (drill 1.016) (layers *.Cu *.Mask))
  (pad 1 thru_hole circle (at 0 2.54) (size 1.524 1.524) (drill 1.016) (layers *.Cu *.Mask))
  (pad 1 thru_hole circle (at 0 0) (size 1.524 1.524) (drill 1.016) (layers *.Cu *.Mask)))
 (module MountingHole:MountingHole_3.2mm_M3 (layer F.Cu) (at 194.31 80.01)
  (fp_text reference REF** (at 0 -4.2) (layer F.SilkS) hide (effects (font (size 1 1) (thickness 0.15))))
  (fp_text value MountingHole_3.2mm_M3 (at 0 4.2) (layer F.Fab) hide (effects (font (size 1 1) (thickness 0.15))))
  (pad 1 np_thru_hole circle (at 0 0) (size 3.2 3.2) (drill 3.2) (layers *.Cu *.Mask)))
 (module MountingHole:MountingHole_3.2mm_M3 (layer F.Cu) (at 229.87 80.01)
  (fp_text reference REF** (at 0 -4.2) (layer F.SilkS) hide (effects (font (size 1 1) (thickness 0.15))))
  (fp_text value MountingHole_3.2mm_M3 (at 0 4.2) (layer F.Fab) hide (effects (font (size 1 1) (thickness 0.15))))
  (pad 1 np_thru_hole circle (at 0 0) (size 3.2 3.2) (drill 3.2) (layers *.Cu *.Mask)))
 (gr_line (start 187.96 99.06) (end 236.22 99.06) (layer Edge.Cuts) (width 0.05))
 (gr_line (start 187.96 60.96) (end 236.22 60.96) (layer Edge.Cuts) (width 0.05))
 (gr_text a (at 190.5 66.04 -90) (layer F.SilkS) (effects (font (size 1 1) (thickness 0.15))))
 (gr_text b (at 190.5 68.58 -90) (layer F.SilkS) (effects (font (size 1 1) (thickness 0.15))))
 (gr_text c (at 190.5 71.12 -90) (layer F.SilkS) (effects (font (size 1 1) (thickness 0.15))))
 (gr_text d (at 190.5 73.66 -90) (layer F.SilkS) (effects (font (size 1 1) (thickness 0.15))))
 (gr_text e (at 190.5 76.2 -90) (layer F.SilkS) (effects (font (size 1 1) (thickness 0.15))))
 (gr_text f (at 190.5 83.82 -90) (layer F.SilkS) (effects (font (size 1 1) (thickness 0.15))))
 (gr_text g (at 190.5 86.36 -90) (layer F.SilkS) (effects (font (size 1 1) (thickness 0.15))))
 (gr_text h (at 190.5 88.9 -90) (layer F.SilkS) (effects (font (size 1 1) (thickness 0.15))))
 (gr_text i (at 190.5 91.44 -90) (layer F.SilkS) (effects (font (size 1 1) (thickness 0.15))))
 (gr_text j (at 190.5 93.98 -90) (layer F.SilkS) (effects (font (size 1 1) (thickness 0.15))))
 (gr_line (start 187.96 60.96) (end 187.96 99.06) (layer Edge.Cuts) (width 0.05))
 (gr_line (start 236.22 60.96) (end 236.22 99.06) (layer Edge.Cuts) (width 0.1))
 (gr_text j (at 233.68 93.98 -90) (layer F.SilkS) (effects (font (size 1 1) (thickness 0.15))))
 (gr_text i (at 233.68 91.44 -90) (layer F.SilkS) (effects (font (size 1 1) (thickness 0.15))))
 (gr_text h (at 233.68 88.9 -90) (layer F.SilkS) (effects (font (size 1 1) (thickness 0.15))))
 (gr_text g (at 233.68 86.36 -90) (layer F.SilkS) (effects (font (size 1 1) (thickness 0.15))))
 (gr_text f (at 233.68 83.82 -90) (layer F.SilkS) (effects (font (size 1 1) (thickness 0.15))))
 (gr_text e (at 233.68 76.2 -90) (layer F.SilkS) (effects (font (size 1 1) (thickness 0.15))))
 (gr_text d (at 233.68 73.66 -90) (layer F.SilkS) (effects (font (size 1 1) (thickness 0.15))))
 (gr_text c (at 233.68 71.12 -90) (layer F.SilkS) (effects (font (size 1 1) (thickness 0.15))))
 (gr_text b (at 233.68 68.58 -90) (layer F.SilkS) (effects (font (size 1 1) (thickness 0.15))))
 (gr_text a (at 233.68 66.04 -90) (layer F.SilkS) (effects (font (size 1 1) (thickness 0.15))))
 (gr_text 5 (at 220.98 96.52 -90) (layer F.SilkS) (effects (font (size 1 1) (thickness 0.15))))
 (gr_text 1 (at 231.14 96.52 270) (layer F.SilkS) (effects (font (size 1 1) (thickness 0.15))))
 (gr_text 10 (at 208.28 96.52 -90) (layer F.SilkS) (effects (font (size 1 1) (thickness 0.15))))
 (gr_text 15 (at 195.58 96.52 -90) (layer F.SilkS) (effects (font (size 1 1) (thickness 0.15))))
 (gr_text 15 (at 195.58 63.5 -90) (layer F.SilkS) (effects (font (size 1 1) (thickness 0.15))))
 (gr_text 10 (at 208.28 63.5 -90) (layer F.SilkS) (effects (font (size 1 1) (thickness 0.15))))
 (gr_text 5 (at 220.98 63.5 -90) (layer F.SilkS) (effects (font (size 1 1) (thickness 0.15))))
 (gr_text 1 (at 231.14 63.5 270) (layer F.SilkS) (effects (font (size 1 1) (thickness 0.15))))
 (segment (start 203.2 66.04) (end 203.2 76.2) (width 0.4064) (layer F.Cu) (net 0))
 (segment (start 193.04 66.04) (end 193.04 76.2) (width 0.4064) (layer F.Cu) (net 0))
 (segment (start 200.66 66.04) (end 200.66 76.2) (width 0.4064) (layer F.Cu) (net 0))
 (segment (start 205.74 66.04) (end 205.74 76.2) (width 0.4064) (layer F.Cu) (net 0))
 (segment (start 195.58 66.04) (end 195.58 76.2) (width 0.4064) (layer F.Cu) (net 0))
 (segment (start 208.28 66.04) (end 208.28 76.2) (width 0.4064) (layer F.Cu) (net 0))
 (segment (start 198.12 66.04) (end 198.12 76.2) (width 0.4064) (layer F.Cu) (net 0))
 (segment (start 210.82 66.04) (end 210.82 76.2) (width 0.4064) (layer F.Cu) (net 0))
 (segment (start 215.9 66.04) (end 215.9 76.2) (width 0.4064) (layer F.Cu) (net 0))
 (segment (start 218.44 66.04) (end 218.44 76.2) (width 0.4064) (layer F.Cu) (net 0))
 (segment (start 220.98 66.04) (end 220.98 76.2) (width 0.4064) (layer F.Cu) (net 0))
 (segment (start 228.6 66.04) (end 228.6 76.2) (width 0.4064) (layer F.Cu) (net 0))
 (segment (start 223.52 66.04) (end 223.52 76.2) (width 0.4064) (layer F.Cu) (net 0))
 (segment (start 213.36 66.04) (end 213.36 76.2) (width 0.4064) (layer F.Cu) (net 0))
 (segment (start 231.14 66.04) (end 231.14 76.2) (width 0.4064) (layer F.Cu) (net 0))
 (segment (start 226.06 66.04) (end 226.06 76.2) (width 0.4064) (layer F.Cu) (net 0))
 (segment (start 195.58 83.82) (end 195.58 93.98) (width 0.4064) (layer F.Cu) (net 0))
 (segment (start 213.36 83.82) (end 213.36 93.98) (width 0.4064) (layer F.Cu) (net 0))
 (segment (start 220.98 83.82) (end 220.98 93.98) (width 0.4064) (layer F.Cu) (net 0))
 (segment (start 228.6 83.82) (end 228.6 93.98) (width 0.4064) (layer F.Cu) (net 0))
 (segment (start 198.12 83.82) (end 198.12 93.98) (width 0.4064) (layer F.Cu) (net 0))
 (segment (start 218.44 83.82) (end 218.44 93.98) (width 0.4064) (layer F.Cu) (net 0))
 (segment (start 200.66 83.82) (end 200.66 93.98) (width 0.4064) (layer F.Cu) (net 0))
 (segment (start 208.28 83.82) (end 208.28 93.98) (width 0.4064) (layer F.Cu) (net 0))
 (segment (start 203.2 83.82) (end 203.2 93.98) (width 0.4064) (layer F.Cu) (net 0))
 (segment (start 231.14 83.82) (end 231.14 93.98) (width 0.4064) (layer F.Cu) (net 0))
 (segment (start 226.06 83.82) (end 226.06 93.98) (width 0.4064) (layer F.Cu) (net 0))
 (segment (start 193.04 83.82) (end 193.04 93.98) (width 0.4064) (layer F.Cu) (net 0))
 (segment (start 210.82 83.82) (end 210.82 93.98) (width 0.4064) (layer F.Cu) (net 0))
 (segment (start 205.74 83.82) (end 205.74 93.98) (width 0.4064) (layer F.Cu) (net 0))
 (segment (start 223.52 83.82) (end 223.52 93.98) (width 0.4064) (layer F.Cu) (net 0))
 (segment (start 215.9 83.82) (end 215.9 93.98) (width 0.4064) (layer F.Cu) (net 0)))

